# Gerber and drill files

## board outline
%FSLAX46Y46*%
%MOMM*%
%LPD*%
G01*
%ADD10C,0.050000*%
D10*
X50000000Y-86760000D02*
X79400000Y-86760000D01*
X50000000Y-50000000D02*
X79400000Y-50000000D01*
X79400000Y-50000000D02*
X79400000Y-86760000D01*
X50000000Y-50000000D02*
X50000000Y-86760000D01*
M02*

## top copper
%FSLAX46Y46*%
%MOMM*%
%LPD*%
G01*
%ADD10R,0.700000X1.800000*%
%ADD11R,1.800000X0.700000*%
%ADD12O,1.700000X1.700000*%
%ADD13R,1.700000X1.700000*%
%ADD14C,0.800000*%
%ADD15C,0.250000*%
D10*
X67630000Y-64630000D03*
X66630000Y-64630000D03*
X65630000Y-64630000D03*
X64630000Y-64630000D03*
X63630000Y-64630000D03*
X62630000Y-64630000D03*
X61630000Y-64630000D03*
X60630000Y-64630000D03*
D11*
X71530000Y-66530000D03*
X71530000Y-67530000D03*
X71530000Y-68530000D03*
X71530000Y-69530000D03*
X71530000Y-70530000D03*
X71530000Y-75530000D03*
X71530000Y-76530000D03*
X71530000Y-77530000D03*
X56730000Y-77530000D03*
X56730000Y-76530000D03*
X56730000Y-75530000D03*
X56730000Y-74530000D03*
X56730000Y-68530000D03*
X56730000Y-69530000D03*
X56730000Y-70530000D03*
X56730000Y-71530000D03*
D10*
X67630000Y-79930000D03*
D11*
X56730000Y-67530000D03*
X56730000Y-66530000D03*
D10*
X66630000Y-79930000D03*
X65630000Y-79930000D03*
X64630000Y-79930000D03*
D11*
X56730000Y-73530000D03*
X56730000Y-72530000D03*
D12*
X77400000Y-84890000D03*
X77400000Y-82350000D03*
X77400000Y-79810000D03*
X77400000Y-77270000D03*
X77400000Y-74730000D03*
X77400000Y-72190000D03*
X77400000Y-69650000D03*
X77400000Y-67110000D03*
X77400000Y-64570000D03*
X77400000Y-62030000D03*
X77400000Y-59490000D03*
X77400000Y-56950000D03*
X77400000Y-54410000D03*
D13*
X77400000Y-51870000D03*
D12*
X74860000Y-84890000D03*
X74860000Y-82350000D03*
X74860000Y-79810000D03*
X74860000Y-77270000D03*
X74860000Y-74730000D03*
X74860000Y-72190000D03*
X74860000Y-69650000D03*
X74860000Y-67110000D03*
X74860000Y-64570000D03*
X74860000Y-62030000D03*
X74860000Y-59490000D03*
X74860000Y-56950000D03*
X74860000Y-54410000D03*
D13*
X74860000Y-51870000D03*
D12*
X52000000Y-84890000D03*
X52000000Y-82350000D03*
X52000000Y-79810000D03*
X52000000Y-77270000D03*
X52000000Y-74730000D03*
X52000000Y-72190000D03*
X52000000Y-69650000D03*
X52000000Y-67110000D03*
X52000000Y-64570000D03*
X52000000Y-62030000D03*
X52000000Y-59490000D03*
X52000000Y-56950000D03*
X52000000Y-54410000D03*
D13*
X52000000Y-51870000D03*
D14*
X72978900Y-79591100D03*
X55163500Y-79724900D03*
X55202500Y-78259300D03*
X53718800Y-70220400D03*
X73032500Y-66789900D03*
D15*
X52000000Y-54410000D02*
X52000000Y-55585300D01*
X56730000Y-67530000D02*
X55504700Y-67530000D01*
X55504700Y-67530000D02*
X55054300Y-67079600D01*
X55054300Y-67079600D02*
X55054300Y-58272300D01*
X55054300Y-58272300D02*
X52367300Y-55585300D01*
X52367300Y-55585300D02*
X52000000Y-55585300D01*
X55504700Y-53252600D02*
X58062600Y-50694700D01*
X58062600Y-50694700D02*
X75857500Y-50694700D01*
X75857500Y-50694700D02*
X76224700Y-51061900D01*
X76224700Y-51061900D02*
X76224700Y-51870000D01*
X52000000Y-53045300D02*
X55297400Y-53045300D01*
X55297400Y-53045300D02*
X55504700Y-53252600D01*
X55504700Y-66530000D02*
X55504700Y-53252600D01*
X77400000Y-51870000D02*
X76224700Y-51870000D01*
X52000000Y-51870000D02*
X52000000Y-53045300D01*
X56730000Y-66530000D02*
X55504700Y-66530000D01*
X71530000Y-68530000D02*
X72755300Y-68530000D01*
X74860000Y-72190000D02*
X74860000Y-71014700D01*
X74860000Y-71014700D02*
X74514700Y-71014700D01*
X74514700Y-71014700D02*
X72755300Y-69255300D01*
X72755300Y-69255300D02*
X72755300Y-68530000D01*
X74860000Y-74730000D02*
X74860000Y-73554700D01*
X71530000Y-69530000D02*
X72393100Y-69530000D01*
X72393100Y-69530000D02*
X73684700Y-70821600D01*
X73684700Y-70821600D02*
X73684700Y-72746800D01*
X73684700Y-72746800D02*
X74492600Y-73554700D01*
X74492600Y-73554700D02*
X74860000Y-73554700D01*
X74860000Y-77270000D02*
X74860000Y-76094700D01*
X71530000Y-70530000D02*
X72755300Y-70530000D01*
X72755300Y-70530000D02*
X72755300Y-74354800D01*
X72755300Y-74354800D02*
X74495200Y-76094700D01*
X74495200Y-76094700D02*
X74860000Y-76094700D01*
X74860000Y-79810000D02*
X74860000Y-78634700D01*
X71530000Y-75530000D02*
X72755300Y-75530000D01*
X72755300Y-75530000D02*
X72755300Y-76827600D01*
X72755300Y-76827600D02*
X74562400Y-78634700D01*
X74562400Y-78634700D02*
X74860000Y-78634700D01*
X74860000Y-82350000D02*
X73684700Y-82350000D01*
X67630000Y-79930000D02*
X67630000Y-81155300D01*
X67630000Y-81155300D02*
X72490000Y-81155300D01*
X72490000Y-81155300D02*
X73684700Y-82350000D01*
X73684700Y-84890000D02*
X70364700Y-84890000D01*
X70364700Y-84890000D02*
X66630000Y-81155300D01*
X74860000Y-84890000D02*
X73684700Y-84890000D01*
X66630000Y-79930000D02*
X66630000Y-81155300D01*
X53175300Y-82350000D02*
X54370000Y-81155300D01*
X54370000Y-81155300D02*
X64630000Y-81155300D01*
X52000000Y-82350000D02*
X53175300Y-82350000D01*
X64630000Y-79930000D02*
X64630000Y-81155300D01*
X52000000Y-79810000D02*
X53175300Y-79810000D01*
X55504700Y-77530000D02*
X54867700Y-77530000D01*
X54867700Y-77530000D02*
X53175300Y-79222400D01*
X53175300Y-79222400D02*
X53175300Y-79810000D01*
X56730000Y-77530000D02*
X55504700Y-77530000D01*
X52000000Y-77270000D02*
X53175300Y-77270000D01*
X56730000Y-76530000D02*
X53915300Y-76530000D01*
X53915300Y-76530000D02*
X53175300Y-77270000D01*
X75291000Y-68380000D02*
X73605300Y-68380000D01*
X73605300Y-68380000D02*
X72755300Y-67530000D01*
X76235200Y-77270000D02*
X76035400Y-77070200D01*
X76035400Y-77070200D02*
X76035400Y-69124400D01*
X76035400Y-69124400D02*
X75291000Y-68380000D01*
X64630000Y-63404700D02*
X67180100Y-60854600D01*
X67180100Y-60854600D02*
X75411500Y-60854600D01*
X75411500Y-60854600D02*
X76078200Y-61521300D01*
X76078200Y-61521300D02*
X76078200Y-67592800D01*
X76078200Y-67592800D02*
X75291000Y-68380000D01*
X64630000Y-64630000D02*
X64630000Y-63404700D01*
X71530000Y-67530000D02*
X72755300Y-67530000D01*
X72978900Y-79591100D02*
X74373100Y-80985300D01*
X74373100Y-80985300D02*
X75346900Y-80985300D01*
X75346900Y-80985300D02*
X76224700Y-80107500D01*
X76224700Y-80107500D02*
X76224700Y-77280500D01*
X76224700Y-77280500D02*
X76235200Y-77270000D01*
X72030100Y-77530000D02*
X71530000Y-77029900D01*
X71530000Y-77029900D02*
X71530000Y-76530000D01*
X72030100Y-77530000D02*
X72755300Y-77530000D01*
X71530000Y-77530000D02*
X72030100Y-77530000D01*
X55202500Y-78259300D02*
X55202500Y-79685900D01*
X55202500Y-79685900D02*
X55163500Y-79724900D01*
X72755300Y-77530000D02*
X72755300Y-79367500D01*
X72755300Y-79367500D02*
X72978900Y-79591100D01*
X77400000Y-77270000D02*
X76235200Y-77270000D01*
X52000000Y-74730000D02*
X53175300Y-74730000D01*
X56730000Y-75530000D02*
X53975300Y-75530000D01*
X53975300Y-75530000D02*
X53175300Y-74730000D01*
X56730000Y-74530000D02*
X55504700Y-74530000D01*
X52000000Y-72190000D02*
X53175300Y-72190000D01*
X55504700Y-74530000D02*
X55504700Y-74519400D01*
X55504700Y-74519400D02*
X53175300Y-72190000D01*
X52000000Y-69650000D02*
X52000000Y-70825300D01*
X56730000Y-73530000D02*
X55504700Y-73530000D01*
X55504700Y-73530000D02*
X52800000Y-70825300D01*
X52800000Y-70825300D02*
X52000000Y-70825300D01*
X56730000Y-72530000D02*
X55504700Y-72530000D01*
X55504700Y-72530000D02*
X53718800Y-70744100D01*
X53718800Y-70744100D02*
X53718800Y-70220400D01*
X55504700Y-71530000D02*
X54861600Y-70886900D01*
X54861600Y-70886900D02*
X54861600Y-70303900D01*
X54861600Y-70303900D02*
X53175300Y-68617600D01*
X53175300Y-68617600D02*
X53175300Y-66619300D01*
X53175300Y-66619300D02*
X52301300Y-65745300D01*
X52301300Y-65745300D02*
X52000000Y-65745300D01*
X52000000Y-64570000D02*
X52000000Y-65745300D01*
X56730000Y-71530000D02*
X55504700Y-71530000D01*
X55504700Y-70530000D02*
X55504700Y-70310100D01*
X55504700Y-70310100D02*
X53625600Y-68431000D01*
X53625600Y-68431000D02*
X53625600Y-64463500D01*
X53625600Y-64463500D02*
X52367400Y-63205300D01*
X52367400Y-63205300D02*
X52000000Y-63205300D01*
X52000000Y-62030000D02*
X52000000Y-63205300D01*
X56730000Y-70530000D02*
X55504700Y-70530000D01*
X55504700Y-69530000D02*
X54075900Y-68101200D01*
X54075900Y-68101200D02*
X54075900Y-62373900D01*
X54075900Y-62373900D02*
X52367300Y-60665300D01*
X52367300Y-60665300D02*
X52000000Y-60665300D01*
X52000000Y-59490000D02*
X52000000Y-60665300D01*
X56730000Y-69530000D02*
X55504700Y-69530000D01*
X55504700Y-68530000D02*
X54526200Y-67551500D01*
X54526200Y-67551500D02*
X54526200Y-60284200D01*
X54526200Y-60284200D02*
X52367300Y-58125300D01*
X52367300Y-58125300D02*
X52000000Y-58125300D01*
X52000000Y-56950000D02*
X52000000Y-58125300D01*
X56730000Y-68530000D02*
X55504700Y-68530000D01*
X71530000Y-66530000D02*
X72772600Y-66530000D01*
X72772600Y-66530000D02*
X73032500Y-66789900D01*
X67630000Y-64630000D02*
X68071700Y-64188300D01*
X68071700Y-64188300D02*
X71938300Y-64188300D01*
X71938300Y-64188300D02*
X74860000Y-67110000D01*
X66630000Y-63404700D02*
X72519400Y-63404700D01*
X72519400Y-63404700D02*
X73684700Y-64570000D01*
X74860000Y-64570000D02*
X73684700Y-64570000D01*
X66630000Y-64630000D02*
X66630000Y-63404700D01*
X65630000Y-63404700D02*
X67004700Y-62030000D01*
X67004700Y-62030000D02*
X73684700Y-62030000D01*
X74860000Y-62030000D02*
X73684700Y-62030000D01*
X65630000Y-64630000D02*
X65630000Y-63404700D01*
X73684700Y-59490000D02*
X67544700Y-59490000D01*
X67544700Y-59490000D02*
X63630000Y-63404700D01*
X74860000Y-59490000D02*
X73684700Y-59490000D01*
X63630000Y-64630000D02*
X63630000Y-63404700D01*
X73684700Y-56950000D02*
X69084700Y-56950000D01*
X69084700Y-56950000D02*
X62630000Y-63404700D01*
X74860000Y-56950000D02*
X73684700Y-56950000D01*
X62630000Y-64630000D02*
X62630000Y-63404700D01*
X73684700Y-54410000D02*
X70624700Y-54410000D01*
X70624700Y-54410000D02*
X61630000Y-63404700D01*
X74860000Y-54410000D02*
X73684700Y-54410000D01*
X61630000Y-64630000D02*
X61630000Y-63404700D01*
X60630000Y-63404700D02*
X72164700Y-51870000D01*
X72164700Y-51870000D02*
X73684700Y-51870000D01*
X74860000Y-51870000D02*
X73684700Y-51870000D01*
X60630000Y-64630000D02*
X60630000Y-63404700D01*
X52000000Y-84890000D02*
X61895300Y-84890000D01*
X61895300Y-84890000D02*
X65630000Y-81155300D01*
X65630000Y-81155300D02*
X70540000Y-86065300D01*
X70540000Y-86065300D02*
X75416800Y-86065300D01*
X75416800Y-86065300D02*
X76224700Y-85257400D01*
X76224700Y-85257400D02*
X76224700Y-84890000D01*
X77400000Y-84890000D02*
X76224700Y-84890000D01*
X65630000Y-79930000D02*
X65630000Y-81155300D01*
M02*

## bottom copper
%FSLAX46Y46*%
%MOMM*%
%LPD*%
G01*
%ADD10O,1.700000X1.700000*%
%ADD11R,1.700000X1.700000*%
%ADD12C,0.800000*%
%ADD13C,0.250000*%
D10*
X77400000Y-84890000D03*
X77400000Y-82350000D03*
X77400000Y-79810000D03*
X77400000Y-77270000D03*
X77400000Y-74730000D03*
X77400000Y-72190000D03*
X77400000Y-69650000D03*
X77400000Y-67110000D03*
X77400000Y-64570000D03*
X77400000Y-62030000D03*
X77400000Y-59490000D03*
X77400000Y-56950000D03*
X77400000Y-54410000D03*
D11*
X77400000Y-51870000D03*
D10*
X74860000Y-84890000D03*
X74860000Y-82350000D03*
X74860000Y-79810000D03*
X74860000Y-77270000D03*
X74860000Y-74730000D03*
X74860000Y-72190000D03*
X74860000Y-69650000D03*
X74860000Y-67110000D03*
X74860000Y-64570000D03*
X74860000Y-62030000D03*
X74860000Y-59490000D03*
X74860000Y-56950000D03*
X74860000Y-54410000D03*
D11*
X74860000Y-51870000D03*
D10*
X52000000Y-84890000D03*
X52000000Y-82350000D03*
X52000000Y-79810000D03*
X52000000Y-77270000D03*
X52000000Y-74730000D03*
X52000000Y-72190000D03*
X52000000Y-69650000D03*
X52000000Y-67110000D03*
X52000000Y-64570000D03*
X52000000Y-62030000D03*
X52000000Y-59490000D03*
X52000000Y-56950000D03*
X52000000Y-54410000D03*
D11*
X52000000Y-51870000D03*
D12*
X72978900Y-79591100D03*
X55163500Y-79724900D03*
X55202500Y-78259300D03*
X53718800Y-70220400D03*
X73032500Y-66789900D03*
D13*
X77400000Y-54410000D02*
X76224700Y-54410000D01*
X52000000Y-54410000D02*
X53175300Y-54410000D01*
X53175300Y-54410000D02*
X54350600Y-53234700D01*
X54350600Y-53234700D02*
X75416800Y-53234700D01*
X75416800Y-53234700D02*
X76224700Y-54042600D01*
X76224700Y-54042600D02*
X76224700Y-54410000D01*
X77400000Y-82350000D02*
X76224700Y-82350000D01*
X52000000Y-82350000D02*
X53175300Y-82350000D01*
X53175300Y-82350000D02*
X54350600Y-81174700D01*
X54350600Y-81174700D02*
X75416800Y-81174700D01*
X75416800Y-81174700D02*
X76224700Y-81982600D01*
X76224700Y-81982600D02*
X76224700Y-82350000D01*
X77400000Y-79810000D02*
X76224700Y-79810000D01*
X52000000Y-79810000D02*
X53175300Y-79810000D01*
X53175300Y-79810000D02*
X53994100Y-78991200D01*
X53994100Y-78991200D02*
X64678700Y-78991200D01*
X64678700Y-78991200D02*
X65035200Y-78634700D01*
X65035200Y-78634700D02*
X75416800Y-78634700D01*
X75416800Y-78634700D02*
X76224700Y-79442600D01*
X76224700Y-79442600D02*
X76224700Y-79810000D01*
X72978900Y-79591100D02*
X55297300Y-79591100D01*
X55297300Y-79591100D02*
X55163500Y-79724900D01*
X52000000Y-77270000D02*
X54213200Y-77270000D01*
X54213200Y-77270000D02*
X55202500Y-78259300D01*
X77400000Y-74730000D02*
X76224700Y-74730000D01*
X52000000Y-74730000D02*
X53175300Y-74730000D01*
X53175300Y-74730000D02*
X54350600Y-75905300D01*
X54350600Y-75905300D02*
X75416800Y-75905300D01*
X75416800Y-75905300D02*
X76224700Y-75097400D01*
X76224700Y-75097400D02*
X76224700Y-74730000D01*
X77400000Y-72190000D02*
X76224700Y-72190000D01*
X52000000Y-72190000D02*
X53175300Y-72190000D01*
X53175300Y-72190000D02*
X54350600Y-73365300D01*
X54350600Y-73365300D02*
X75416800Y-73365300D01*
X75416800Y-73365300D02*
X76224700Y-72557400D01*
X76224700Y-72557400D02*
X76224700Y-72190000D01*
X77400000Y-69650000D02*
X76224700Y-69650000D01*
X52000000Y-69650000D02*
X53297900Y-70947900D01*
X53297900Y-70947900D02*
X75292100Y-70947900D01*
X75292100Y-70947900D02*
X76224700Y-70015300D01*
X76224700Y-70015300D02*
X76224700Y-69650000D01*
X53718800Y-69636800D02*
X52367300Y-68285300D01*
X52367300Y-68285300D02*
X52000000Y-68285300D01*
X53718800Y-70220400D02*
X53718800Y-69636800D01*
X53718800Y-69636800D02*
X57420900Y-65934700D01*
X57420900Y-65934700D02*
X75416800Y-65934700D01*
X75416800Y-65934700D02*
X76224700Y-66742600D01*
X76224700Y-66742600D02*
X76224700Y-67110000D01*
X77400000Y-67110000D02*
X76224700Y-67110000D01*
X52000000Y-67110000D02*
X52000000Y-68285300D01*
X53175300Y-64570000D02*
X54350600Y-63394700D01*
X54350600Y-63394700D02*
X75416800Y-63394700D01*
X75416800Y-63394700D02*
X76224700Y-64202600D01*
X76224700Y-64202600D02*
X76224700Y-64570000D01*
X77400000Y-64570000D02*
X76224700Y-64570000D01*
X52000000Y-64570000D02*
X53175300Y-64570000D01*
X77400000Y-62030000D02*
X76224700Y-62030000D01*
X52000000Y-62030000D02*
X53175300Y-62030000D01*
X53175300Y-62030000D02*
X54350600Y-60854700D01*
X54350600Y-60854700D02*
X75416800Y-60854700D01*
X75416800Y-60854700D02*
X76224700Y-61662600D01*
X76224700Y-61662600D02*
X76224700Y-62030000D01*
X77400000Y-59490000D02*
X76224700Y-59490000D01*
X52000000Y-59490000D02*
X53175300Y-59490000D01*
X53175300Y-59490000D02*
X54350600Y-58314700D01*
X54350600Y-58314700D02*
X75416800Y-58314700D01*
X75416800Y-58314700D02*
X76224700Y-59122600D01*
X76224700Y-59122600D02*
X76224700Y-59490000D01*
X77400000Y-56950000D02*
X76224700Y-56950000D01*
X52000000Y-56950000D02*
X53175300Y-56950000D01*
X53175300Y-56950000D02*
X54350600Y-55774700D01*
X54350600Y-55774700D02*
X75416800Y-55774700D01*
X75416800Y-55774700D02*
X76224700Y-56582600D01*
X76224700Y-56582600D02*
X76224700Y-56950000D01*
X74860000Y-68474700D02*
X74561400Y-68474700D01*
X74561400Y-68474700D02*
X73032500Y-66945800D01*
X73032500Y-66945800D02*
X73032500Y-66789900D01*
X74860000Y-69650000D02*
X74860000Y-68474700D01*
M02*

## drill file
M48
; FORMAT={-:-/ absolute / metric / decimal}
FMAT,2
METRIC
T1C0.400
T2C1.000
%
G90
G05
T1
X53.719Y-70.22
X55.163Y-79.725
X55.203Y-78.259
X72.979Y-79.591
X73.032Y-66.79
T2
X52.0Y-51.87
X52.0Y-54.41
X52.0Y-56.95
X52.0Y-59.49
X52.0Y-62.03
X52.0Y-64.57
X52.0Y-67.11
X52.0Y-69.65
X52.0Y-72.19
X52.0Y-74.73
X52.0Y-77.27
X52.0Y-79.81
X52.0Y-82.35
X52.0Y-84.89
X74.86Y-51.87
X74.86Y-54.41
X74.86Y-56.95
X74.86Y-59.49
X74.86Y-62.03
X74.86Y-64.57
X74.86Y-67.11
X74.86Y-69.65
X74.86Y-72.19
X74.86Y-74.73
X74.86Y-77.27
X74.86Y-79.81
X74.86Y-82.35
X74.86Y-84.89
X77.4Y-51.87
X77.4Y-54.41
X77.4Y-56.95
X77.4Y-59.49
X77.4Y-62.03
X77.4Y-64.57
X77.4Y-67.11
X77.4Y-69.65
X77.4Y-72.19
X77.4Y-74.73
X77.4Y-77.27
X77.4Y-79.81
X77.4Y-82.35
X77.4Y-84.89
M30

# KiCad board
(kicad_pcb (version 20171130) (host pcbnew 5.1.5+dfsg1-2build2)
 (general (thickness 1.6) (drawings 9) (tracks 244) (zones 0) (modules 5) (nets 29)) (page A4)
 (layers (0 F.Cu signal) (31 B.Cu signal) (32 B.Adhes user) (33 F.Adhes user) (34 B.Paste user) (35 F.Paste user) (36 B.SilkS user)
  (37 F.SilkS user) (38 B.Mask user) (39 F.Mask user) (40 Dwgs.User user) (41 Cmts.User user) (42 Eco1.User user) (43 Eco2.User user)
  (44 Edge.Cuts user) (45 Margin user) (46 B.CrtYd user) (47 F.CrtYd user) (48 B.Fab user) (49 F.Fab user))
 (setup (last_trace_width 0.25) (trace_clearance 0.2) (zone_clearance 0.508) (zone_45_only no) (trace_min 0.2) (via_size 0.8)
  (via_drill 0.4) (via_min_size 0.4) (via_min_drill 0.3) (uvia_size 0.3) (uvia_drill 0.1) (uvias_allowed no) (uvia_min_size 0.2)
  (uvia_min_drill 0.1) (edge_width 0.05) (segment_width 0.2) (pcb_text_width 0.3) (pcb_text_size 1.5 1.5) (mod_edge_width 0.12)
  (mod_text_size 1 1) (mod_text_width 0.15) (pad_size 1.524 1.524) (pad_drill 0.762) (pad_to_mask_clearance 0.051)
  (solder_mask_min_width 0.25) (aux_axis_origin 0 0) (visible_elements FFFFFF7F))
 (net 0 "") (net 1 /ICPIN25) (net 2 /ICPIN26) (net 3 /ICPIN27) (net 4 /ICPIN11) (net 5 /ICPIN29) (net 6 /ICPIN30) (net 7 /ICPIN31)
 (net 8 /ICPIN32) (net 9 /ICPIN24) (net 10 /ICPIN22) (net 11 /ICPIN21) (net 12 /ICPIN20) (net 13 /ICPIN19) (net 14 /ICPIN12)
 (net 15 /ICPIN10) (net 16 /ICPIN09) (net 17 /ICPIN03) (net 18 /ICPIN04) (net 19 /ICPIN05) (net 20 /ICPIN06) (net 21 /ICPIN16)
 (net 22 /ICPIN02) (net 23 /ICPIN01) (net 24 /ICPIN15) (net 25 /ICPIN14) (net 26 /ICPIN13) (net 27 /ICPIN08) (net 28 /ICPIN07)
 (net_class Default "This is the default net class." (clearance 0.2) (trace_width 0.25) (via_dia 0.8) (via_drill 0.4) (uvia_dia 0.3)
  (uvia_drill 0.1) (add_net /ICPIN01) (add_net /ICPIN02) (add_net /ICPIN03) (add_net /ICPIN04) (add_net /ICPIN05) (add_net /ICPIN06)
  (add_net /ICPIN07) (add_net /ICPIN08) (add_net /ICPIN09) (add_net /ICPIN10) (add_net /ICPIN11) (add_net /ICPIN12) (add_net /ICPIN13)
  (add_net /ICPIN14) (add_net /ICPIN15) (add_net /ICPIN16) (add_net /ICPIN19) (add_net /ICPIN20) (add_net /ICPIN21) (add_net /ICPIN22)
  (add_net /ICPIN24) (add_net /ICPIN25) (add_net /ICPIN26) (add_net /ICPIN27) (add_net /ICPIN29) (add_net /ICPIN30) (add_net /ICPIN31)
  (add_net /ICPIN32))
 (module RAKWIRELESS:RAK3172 (layer F.Cu) (at 64.13 72.28)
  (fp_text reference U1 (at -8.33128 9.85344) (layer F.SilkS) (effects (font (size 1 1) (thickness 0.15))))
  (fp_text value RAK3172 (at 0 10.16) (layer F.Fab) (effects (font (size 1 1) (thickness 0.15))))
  (pad 25 smd rect (at 3.5 -7.65 270) (size 1.8 0.7) (layers F.Cu F.Paste F.Mask) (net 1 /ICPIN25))
  (pad 26 smd rect (at 2.5 -7.65 270) (size 1.8 0.7) (layers F.Cu F.Paste F.Mask) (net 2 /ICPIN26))
  (pad 27 smd rect (at 1.5 -7.65 270) (size 1.8 0.7) (layers F.Cu F.Paste F.Mask) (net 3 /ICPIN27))
  (pad 28 smd rect (at 0.5 -7.65 270) (size 1.8 0.7) (layers F.Cu F.Paste F.Mask) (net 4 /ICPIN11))
  (pad 29 smd rect (at -0.5 -7.65 270) (size 1.8 0.7) (layers F.Cu F.Paste F.Mask) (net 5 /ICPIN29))
  (pad 30 smd rect (at -1.5 -7.65 270) (size 1.8 0.7) (layers F.Cu F.Paste F.Mask) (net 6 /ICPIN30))
  (pad 31 smd rect (at -2.5 -7.65 270) (size 1.8 0.7) (layers F.Cu F.Paste F.Mask) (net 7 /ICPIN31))
  (pad 32 smd rect (at -3.5 -7.65 270) (size 1.8 0.7) (layers F.Cu F.Paste F.Mask) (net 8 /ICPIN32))
  (pad 24 smd rect (at 7.4 -5.75) (size 1.8 0.7) (layers F.Cu F.Paste F.Mask) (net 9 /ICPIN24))
  (pad 23 smd rect (at 7.4 -4.75) (size 1.8 0.7) (layers F.Cu F.Paste F.Mask) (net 4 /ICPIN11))
  (pad 22 smd rect (at 7.4 -3.75) (size 1.8 0.7) (layers F.Cu F.Paste F.Mask) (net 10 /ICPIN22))
  (pad 21 smd rect (at 7.4 -2.75) (size 1.8 0.7) (layers F.Cu F.Paste F.Mask) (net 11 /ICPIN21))
  (pad 20 smd rect (at 7.4 -1.75) (size 1.8 0.7) (layers F.Cu F.Paste F.Mask) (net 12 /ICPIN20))
  (pad 19 smd rect (at 7.4 3.25) (size 1.8 0.7) (layers F.Cu F.Paste F.Mask) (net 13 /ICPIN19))
  (pad 18 smd rect (at 7.4 4.25) (size 1.8 0.7) (layers F.Cu F.Paste F.Mask) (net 4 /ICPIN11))
  (pad 17 smd rect (at 7.4 5.25) (size 1.8 0.7) (layers F.Cu F.Paste F.Mask) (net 4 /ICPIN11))
  (pad 12 smd rect (at -7.4 5.25) (size 1.8 0.7) (layers F.Cu F.Paste F.Mask) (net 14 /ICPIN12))
  (pad 11 smd rect (at -7.4 4.25) (size 1.8 0.7) (layers F.Cu F.Paste F.Mask) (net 4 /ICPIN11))
  (pad 10 smd rect (at -7.4 3.25) (size 1.8 0.7) (layers F.Cu F.Paste F.Mask) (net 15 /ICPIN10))
  (pad 9 smd rect (at -7.4 2.25) (size 1.8 0.7) (layers F.Cu F.Paste F.Mask) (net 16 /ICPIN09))
  (pad 3 smd rect (at -7.4 -3.75) (size 1.8 0.7) (layers F.Cu F.Paste F.Mask) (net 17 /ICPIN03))
  (pad 4 smd rect (at -7.4 -2.75) (size 1.8 0.7) (layers F.Cu F.Paste F.Mask) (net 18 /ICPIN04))
  (pad 5 smd rect (at -7.4 -1.75) (size 1.8 0.7) (layers F.Cu F.Paste F.Mask) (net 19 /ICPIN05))
  (pad 6 smd rect (at -7.4 -0.75) (size 1.8 0.7) (layers F.Cu F.Paste F.Mask) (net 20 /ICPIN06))
  (pad 16 smd rect (at 3.5 7.65 90) (size 1.8 0.7) (layers F.Cu F.Paste F.Mask) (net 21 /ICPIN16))
  (pad 2 smd rect (at -7.4 -4.75) (size 1.8 0.7) (layers F.Cu F.Paste F.Mask) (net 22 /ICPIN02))
  (pad 1 smd rect (at -7.4 -5.75) (size 1.8 0.7) (layers F.Cu F.Paste F.Mask) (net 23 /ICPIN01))
  (pad 15 smd rect (at 2.5 7.65 90) (size 1.8 0.7) (layers F.Cu F.Paste F.Mask) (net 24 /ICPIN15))
  (pad 14 smd rect (at 1.5 7.65 90) (size 1.8 0.7) (layers F.Cu F.Paste F.Mask) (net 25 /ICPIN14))
  (pad 13 smd rect (at 0.5 7.65 270) (size 1.8 0.7) (layers F.Cu F.Paste F.Mask) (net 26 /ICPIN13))
  (pad 8 smd rect (at -7.4 1.25) (size 1.8 0.7) (layers F.Cu F.Paste F.Mask) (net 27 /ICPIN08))
  (pad 7 smd rect (at -7.4 0.25) (size 1.8 0.7) (layers F.Cu F.Paste F.Mask) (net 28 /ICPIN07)))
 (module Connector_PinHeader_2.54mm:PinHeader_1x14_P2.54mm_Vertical (layer F.Cu) (at 77.4 51.87)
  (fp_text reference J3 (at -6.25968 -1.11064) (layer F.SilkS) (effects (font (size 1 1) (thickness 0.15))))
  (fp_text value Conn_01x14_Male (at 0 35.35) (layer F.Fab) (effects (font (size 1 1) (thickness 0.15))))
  (pad 14 thru_hole oval (at 0 33.02) (size 1.7 1.7) (drill 1) (layers *.Cu *.Mask) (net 25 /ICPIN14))
  (pad 13 thru_hole oval (at 0 30.48) (size 1.7 1.7) (drill 1) (layers *.Cu *.Mask) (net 26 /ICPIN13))
  (pad 12 thru_hole oval (at 0 27.94) (size 1.7 1.7) (drill 1) (layers *.Cu *.Mask) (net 14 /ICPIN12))
  (pad 11 thru_hole oval (at 0 25.4) (size 1.7 1.7) (drill 1) (layers *.Cu *.Mask) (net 4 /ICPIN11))
  (pad 10 thru_hole oval (at 0 22.86) (size 1.7 1.7) (drill 1) (layers *.Cu *.Mask) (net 15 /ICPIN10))
  (pad 9 thru_hole oval (at 0 20.32) (size 1.7 1.7) (drill 1) (layers *.Cu *.Mask) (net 16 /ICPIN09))
  (pad 8 thru_hole oval (at 0 17.78) (size 1.7 1.7) (drill 1) (layers *.Cu *.Mask) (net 27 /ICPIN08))
  (pad 7 thru_hole oval (at 0 15.24) (size 1.7 1.7) (drill 1) (layers *.Cu *.Mask) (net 28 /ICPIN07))
  (pad 6 thru_hole oval (at 0 12.7) (size 1.7 1.7) (drill 1) (layers *.Cu *.Mask) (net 20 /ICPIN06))
  (pad 5 thru_hole oval (at 0 10.16) (size 1.7 1.7) (drill 1) (layers *.Cu *.Mask) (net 19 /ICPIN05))
  (pad 4 thru_hole oval (at 0 7.62) (size 1.7 1.7) (drill 1) (layers *.Cu *.Mask) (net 18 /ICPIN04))
  (pad 3 thru_hole oval (at 0 5.08) (size 1.7 1.7) (drill 1) (layers *.Cu *.Mask) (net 17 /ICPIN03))
  (pad 2 thru_hole oval (at 0 2.54) (size 1.7 1.7) (drill 1) (layers *.Cu *.Mask) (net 22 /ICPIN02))
  (pad 1 thru_hole rect (at 0 0) (size 1.7 1.7) (drill 1) (layers *.Cu *.Mask) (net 23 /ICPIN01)))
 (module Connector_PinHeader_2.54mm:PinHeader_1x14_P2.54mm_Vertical (layer F.Cu) (at 74.86 51.87)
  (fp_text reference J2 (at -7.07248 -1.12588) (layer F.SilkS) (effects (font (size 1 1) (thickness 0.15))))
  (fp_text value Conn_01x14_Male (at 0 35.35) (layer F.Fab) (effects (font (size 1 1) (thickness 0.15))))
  (pad 14 thru_hole oval (at 0 33.02) (size 1.7 1.7) (drill 1) (layers *.Cu *.Mask) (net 24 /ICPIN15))
  (pad 13 thru_hole oval (at 0 30.48) (size 1.7 1.7) (drill 1) (layers *.Cu *.Mask) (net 21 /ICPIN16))
  (pad 12 thru_hole oval (at 0 27.94) (size 1.7 1.7) (drill 1) (layers *.Cu *.Mask) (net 13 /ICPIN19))
  (pad 11 thru_hole oval (at 0 25.4) (size 1.7 1.7) (drill 1) (layers *.Cu *.Mask) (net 12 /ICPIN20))
  (pad 10 thru_hole oval (at 0 22.86) (size 1.7 1.7) (drill 1) (layers *.Cu *.Mask) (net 11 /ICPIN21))
  (pad 9 thru_hole oval (at 0 20.32) (size 1.7 1.7) (drill 1) (layers *.Cu *.Mask) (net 10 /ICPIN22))
  (pad 8 thru_hole oval (at 0 17.78) (size 1.7 1.7) (drill 1) (layers *.Cu *.Mask) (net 9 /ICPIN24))
  (pad 7 thru_hole oval (at 0 15.24) (size 1.7 1.7) (drill 1) (layers *.Cu *.Mask) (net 1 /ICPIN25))
  (pad 6 thru_hole oval (at 0 12.7) (size 1.7 1.7) (drill 1) (layers *.Cu *.Mask) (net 2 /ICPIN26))
  (pad 5 thru_hole oval (at 0 10.16) (size 1.7 1.7) (drill 1) (layers *.Cu *.Mask) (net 3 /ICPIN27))
  (pad 4 thru_hole oval (at 0 7.62) (size 1.7 1.7) (drill 1) (layers *.Cu *.Mask) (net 5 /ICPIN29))
  (pad 3 thru_hole oval (at 0 5.08) (size 1.7 1.7) (drill 1) (layers *.Cu *.Mask) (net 6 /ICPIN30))
  (pad 2 thru_hole oval (at 0 2.54) (size 1.7 1.7) (drill 1) (layers *.Cu *.Mask) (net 7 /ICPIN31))
  (pad 1 thru_hole rect (at 0 0) (size 1.7 1.7) (drill 1) (layers *.Cu *.Mask) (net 8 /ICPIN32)))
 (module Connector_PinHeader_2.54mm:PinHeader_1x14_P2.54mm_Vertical (layer F.Cu) (at 52 51.87)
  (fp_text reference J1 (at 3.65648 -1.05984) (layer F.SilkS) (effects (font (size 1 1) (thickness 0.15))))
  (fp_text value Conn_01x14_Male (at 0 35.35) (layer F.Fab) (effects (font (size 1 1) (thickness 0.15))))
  (pad 14 thru_hole oval (at 0 33.02) (size 1.7 1.7) (drill 1) (layers *.Cu *.Mask) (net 25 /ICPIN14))
  (pad 13 thru_hole oval (at 0 30.48) (size 1.7 1.7) (drill 1) (layers *.Cu *.Mask) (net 26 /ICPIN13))
  (pad 12 thru_hole oval (at 0 27.94) (size 1.7 1.7) (drill 1) (layers *.Cu *.Mask) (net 14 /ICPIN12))
  (pad 11 thru_hole oval (at 0 25.4) (size 1.7 1.7) (drill 1) (layers *.Cu *.Mask) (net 4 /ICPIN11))
  (pad 10 thru_hole oval (at 0 22.86) (size 1.7 1.7) (drill 1) (layers *.Cu *.Mask) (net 15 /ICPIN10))
  (pad 9 thru_hole oval (at 0 20.32) (size 1.7 1.7) (drill 1) (layers *.Cu *.Mask) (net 16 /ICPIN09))
  (pad 8 thru_hole oval (at 0 17.78) (size 1.7 1.7) (drill 1) (layers *.Cu *.Mask) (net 27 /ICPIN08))
  (pad 7 thru_hole oval (at 0 15.24) (size 1.7 1.7) (drill 1) (layers *.Cu *.Mask) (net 28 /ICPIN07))
  (pad 6 thru_hole oval (at 0 12.7) (size 1.7 1.7) (drill 1) (layers *.Cu *.Mask) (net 20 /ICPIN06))
  (pad 5 thru_hole oval (at 0 10.16) (size 1.7 1.7) (drill 1) (layers *.Cu *.Mask) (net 19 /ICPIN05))
  (pad 4 thru_hole oval (at 0 7.62) (size 1.7 1.7) (drill 1) (layers *.Cu *.Mask) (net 18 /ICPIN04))
  (pad 3 thru_hole oval (at 0 5.08) (size 1.7 1.7) (drill 1) (layers *.Cu *.Mask) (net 17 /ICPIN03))
  (pad 2 thru_hole oval (at 0 2.54) (size 1.7 1.7) (drill 1) (layers *.Cu *.Mask) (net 22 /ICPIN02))
  (pad 1 thru_hole rect (at 0 0) (size 1.7 1.7) (drill 1) (layers *.Cu *.Mask) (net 23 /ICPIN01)))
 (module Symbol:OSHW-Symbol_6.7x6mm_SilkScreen (layer F.Cu) (at 60.7822 56.03748)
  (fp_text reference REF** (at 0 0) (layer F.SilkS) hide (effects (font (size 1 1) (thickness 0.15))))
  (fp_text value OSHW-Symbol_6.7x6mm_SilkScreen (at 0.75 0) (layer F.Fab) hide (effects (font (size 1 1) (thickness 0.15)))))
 (gr_line (start 50 86.76) (end 79.4 86.76) (layer Edge.Cuts) (width 0.05))
 (gr_line (start 50 50) (end 79.4 50) (layer Edge.Cuts) (width 0.05))
 (gr_line (start 79.4 50) (end 79.4 86.76) (layer Edge.Cuts) (width 0.05))
 (gr_line (start 50 50) (end 50 86.76) (layer Edge.Cuts) (width 0.05))
 (segment (start 52 54.41) (end 52 55.5853) (width 0.25) (layer F.Cu) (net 22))
 (segment (start 56.73 67.53) (end 55.5047 67.53) (width 0.25) (layer F.Cu) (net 22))
 (segment (start 55.5047 67.53) (end 55.0543 67.0796) (width 0.25) (layer F.Cu) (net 22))
 (segment (start 55.0543 67.0796) (end 55.0543 58.2723) (width 0.25) (layer F.Cu) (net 22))
 (segment (start 55.0543 58.2723) (end 52.3673 55.5853) (width 0.25) (layer F.Cu) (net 22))
 (segment (start 52.3673 55.5853) (end 52 55.5853) (width 0.25) (layer F.Cu) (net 22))
 (segment (start 77.4 54.41) (end 76.2247 54.41) (width 0.25) (layer B.Cu) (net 22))
 (segment (start 52 54.41) (end 53.1753 54.41) (width 0.25) (layer B.Cu) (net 22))
 (segment (start 53.1753 54.41) (end 54.3506 53.2347) (width 0.25) (layer B.Cu) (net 22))
 (segment (start 54.3506 53.2347) (end 75.4168 53.2347) (width 0.25) (layer B.Cu) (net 22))
 (segment (start 75.4168 53.2347) (end 76.2247 54.0426) (width 0.25) (layer B.Cu) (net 22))
 (segment (start 76.2247 54.0426) (end 76.2247 54.41) (width 0.25) (layer B.Cu) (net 22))
 (segment (start 55.5047 53.2526) (end 58.0626 50.6947) (width 0.25) (layer F.Cu) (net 23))
 (segment (start 58.0626 50.6947) (end 75.8575 50.6947) (width 0.25) (layer F.Cu) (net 23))
 (segment (start 75.8575 50.6947) (end 76.2247 51.0619) (width 0.25) (layer F.Cu) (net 23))
 (segment (start 76.2247 51.0619) (end 76.2247 51.87) (width 0.25) (layer F.Cu) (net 23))
 (segment (start 52 53.0453) (end 55.2974 53.0453) (width 0.25) (layer F.Cu) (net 23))
 (segment (start 55.2974 53.0453) (end 55.5047 53.2526) (width 0.25) (layer F.Cu) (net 23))
 (segment (start 55.5047 66.53) (end 55.5047 53.2526) (width 0.25) (layer F.Cu) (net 23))
 (segment (start 77.4 51.87) (end 76.2247 51.87) (width 0.25) (layer F.Cu) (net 23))
 (segment (start 52 51.87) (end 52 53.0453) (width 0.25) (layer F.Cu) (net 23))
 (segment (start 56.73 66.53) (end 55.5047 66.53) (width 0.25) (layer F.Cu) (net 23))
 (segment (start 71.53 68.53) (end 72.7553 68.53) (width 0.25) (layer F.Cu) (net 10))
 (segment (start 74.86 72.19) (end 74.86 71.0147) (width 0.25) (layer F.Cu) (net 10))
 (segment (start 74.86 71.0147) (end 74.5147 71.0147) (width 0.25) (layer F.Cu) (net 10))
 (segment (start 74.5147 71.0147) (end 72.7553 69.2553) (width 0.25) (layer F.Cu) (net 10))
 (segment (start 72.7553 69.2553) (end 72.7553 68.53) (width 0.25) (layer F.Cu) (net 10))
 (segment (start 74.86 74.73) (end 74.86 73.5547) (width 0.25) (layer F.Cu) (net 11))
 (segment (start 71.53 69.53) (end 72.3931 69.53) (width 0.25) (layer F.Cu) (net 11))
 (segment (start 72.3931 69.53) (end 73.6847 70.8216) (width 0.25) (layer F.Cu) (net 11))
 (segment (start 73.6847 70.8216) (end 73.6847 72.7468) (width 0.25) (layer F.Cu) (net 11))
 (segment (start 73.6847 72.7468) (end 74.4926 73.5547) (width 0.25) (layer F.Cu) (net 11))
 (segment (start 74.4926 73.5547) (end 74.86 73.5547) (width 0.25) (layer F.Cu) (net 11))
 (segment (start 74.86 77.27) (end 74.86 76.0947) (width 0.25) (layer F.Cu) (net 12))
 (segment (start 71.53 70.53) (end 72.7553 70.53) (width 0.25) (layer F.Cu) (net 12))
 (segment (start 72.7553 70.53) (end 72.7553 74.3548) (width 0.25) (layer F.Cu) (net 12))
 (segment (start 72.7553 74.3548) (end 74.4952 76.0947) (width 0.25) (layer F.Cu) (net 12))
 (segment (start 74.4952 76.0947) (end 74.86 76.0947) (width 0.25) (layer F.Cu) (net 12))
 (segment (start 74.86 79.81) (end 74.86 78.6347) (width 0.25) (layer F.Cu) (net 13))
 (segment (start 71.53 75.53) (end 72.7553 75.53) (width 0.25) (layer F.Cu) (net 13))
 (segment (start 72.7553 75.53) (end 72.7553 76.8276) (width 0.25) (layer F.Cu) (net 13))
 (segment (start 72.7553 76.8276) (end 74.5624 78.6347) (width 0.25) (layer F.Cu) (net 13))
 (segment (start 74.5624 78.6347) (end 74.86 78.6347) (width 0.25) (layer F.Cu) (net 13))
 (segment (start 74.86 82.35) (end 73.6847 82.35) (width 0.25) (layer F.Cu) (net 21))
 (segment (start 67.63 79.93) (end 67.63 81.1553) (width 0.25) (layer F.Cu) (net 21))
 (segment (start 67.63 81.1553) (end 72.49 81.1553) (width 0.25) (layer F.Cu) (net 21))
 (segment (start 72.49 81.1553) (end 73.6847 82.35) (width 0.25) (layer F.Cu) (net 21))
 (segment (start 73.6847 84.89) (end 70.3647 84.89) (width 0.25) (layer F.Cu) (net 24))
 (segment (start 70.3647 84.89) (end 66.63 81.1553) (width 0.25) (layer F.Cu) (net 24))
 (segment (start 74.86 84.89) (end 73.6847 84.89) (width 0.25) (layer F.Cu) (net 24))
 (segment (start 66.63 79.93) (end 66.63 81.1553) (width 0.25) (layer F.Cu) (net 24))
 (segment (start 77.4 82.35) (end 76.2247 82.35) (width 0.25) (layer B.Cu) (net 26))
 (segment (start 52 82.35) (end 53.1753 82.35) (width 0.25) (layer B.Cu) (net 26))
 (segment (start 53.1753 82.35) (end 54.3506 81.1747) (width 0.25) (layer B.Cu) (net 26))
 (segment (start 54.3506 81.1747) (end 75.4168 81.1747) (width 0.25) (layer B.Cu) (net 26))
 (segment (start 75.4168 81.1747) (end 76.2247 81.9826) (width 0.25) (layer B.Cu) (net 26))
 (segment (start 76.2247 81.9826) (end 76.2247 82.35) (width 0.25) (layer B.Cu) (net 26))
 (segment (start 53.1753 82.35) (end 54.37 81.1553) (width 0.25) (layer F.Cu) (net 26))
 (segment (start 54.37 81.1553) (end 64.63 81.1553) (width 0.25) (layer F.Cu) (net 26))
 (segment (start 52 82.35) (end 53.1753 82.35) (width 0.25) (layer F.Cu) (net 26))
 (segment (start 64.63 79.93) (end 64.63 81.1553) (width 0.25) (layer F.Cu) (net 26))
 (segment (start 77.4 79.81) (end 76.2247 79.81) (width 0.25) (layer B.Cu) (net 14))
 (segment (start 52 79.81) (end 53.1753 79.81) (width 0.25) (layer B.Cu) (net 14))
 (segment (start 53.1753 79.81) (end 53.9941 78.9912) (width 0.25) (layer B.Cu) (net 14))
 (segment (start 53.9941 78.9912) (end 64.6787 78.9912) (width 0.25) (layer B.Cu) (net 14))
 (segment (start 64.6787 78.9912) (end 65.0352 78.6347) (width 0.25) (layer B.Cu) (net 14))
 (segment (start 65.0352 78.6347) (end 75.4168 78.6347) (width 0.25) (layer B.Cu) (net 14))
 (segment (start 75.4168 78.6347) (end 76.2247 79.4426) (width 0.25) (layer B.Cu) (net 14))
 (segment (start 76.2247 79.4426) (end 76.2247 79.81) (width 0.25) (layer B.Cu) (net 14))
 (segment (start 52 79.81) (end 53.1753 79.81) (width 0.25) (layer F.Cu) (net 14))
 (segment (start 55.5047 77.53) (end 54.8677 77.53) (width 0.25) (layer F.Cu) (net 14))
 (segment (start 54.8677 77.53) (end 53.1753 79.2224) (width 0.25) (layer F.Cu) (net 14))
 (segment (start 53.1753 79.2224) (end 53.1753 79.81) (width 0.25) (layer F.Cu) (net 14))
 (segment (start 56.73 77.53) (end 55.5047 77.53) (width 0.25) (layer F.Cu) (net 14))
 (segment (start 52 77.27) (end 53.1753 77.27) (width 0.25) (layer F.Cu) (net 4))
 (segment (start 56.73 76.53) (end 53.9153 76.53) (width 0.25) (layer F.Cu) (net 4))
 (segment (start 53.9153 76.53) (end 53.1753 77.27) (width 0.25) (layer F.Cu) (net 4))
 (segment (start 75.291 68.38) (end 73.6053 68.38) (width 0.25) (layer F.Cu) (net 4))
 (segment (start 73.6053 68.38) (end 72.7553 67.53) (width 0.25) (layer F.Cu) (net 4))
 (segment (start 76.2352 77.27) (end 76.0354 77.0702) (width 0.25) (layer F.Cu) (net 4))
 (segment (start 76.0354 77.0702) (end 76.0354 69.1244) (width 0.25) (layer F.Cu) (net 4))
 (segment (start 76.0354 69.1244) (end 75.291 68.38) (width 0.25) (layer F.Cu) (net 4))
 (segment (start 64.63 63.4047) (end 67.1801 60.8546) (width 0.25) (layer F.Cu) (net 4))
 (segment (start 67.1801 60.8546) (end 75.4115 60.8546) (width 0.25) (layer F.Cu) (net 4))
 (segment (start 75.4115 60.8546) (end 76.0782 61.5213) (width 0.25) (layer F.Cu) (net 4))
 (segment (start 76.0782 61.5213) (end 76.0782 67.5928) (width 0.25) (layer F.Cu) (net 4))
 (segment (start 76.0782 67.5928) (end 75.291 68.38) (width 0.25) (layer F.Cu) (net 4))
 (segment (start 64.63 64.63) (end 64.63 63.4047) (width 0.25) (layer F.Cu) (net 4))
 (segment (start 71.53 67.53) (end 72.7553 67.53) (width 0.25) (layer F.Cu) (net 4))
 (segment (start 72.9789 79.5911) (end 74.3731 80.9853) (width 0.25) (layer F.Cu) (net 4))
 (segment (start 74.3731 80.9853) (end 75.3469 80.9853) (width 0.25) (layer F.Cu) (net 4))
 (segment (start 75.3469 80.9853) (end 76.2247 80.1075) (width 0.25) (layer F.Cu) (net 4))
 (segment (start 76.2247 80.1075) (end 76.2247 77.2805) (width 0.25) (layer F.Cu) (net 4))
 (segment (start 76.2247 77.2805) (end 76.2352 77.27) (width 0.25) (layer F.Cu) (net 4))
 (segment (start 72.0301 77.53) (end 71.53 77.0299) (width 0.25) (layer F.Cu) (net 4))
 (segment (start 71.53 77.0299) (end 71.53 76.53) (width 0.25) (layer F.Cu) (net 4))
 (segment (start 72.0301 77.53) (end 72.7553 77.53) (width 0.25) (layer F.Cu) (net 4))
 (segment (start 71.53 77.53) (end 72.0301 77.53) (width 0.25) (layer F.Cu) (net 4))
 (segment (start 55.2025 78.2593) (end 55.2025 79.6859) (width 0.25) (layer F.Cu) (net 4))
 (segment (start 55.2025 79.6859) (end 55.1635 79.7249) (width 0.25) (layer F.Cu) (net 4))
 (segment (start 72.9789 79.5911) (end 55.2973 79.5911) (width 0.25) (layer B.Cu) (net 4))
 (segment (start 55.2973 79.5911) (end 55.1635 79.7249) (width 0.25) (layer B.Cu) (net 4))
 (segment (start 72.7553 77.53) (end 72.7553 79.3675) (width 0.25) (layer F.Cu) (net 4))
 (segment (start 72.7553 79.3675) (end 72.9789 79.5911) (width 0.25) (layer F.Cu) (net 4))
 (segment (start 52 77.27) (end 54.2132 77.27) (width 0.25) (layer B.Cu) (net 4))
 (segment (start 54.2132 77.27) (end 55.2025 78.2593) (width 0.25) (layer B.Cu) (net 4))
 (segment (start 77.4 77.27) (end 76.2352 77.27) (width 0.25) (layer F.Cu) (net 4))
 (via (at 72.9789 79.5911) (size 0.8) (layers F.Cu B.Cu) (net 4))
 (via (at 55.1635 79.7249) (size 0.8) (layers F.Cu B.Cu) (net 4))
 (via (at 55.2025 78.2593) (size 0.8) (layers F.Cu B.Cu) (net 4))
 (segment (start 52 74.73) (end 53.1753 74.73) (width 0.25) (layer F.Cu) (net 15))
 (segment (start 56.73 75.53) (end 53.9753 75.53) (width 0.25) (layer F.Cu) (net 15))
 (segment (start 53.9753 75.53) (end 53.1753 74.73) (width 0.25) (layer F.Cu) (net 15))
 (segment (start 77.4 74.73) (end 76.2247 74.73) (width 0.25) (layer B.Cu) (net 15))
 (segment (start 52 74.73) (end 53.1753 74.73) (width 0.25) (layer B.Cu) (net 15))
 (segment (start 53.1753 74.73) (end 54.3506 75.9053) (width 0.25) (layer B.Cu) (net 15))
 (segment (start 54.3506 75.9053) (end 75.4168 75.9053) (width 0.25) (layer B.Cu) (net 15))
 (segment (start 75.4168 75.9053) (end 76.2247 75.0974) (width 0.25) (layer B.Cu) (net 15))
 (segment (start 76.2247 75.0974) (end 76.2247 74.73) (width 0.25) (layer B.Cu) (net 15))
 (segment (start 77.4 72.19) (end 76.2247 72.19) (width 0.25) (layer B.Cu) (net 16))
 (segment (start 52 72.19) (end 53.1753 72.19) (width 0.25) (layer B.Cu) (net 16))
 (segment (start 53.1753 72.19) (end 54.3506 73.3653) (width 0.25) (layer B.Cu) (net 16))
 (segment (start 54.3506 73.3653) (end 75.4168 73.3653) (width 0.25) (layer B.Cu) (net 16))
 (segment (start 75.4168 73.3653) (end 76.2247 72.5574) (width 0.25) (layer B.Cu) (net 16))
 (segment (start 76.2247 72.5574) (end 76.2247 72.19) (width 0.25) (layer B.Cu) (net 16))
 (segment (start 56.73 74.53) (end 55.5047 74.53) (width 0.25) (layer F.Cu) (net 16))
 (segment (start 52 72.19) (end 53.1753 72.19) (width 0.25) (layer F.Cu) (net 16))
 (segment (start 55.5047 74.53) (end 55.5047 74.5194) (width 0.25) (layer F.Cu) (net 16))
 (segment (start 55.5047 74.5194) (end 53.1753 72.19) (width 0.25) (layer F.Cu) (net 16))
 (segment (start 77.4 69.65) (end 76.2247 69.65) (width 0.25) (layer B.Cu) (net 27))
 (segment (start 52 69.65) (end 53.2979 70.9479) (width 0.25) (layer B.Cu) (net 27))
 (segment (start 53.2979 70.9479) (end 75.2921 70.9479) (width 0.25) (layer B.Cu) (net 27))
 (segment (start 75.2921 70.9479) (end 76.2247 70.0153) (width 0.25) (layer B.Cu) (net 27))
 (segment (start 76.2247 70.0153) (end 76.2247 69.65) (width 0.25) (layer B.Cu) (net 27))
 (segment (start 52 69.65) (end 52 70.8253) (width 0.25) (layer F.Cu) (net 27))
 (segment (start 56.73 73.53) (end 55.5047 73.53) (width 0.25) (layer F.Cu) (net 27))
 (segment (start 55.5047 73.53) (end 52.8 70.8253) (width 0.25) (layer F.Cu) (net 27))
 (segment (start 52.8 70.8253) (end 52 70.8253) (width 0.25) (layer F.Cu) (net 27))
 (segment (start 53.7188 69.6368) (end 52.3673 68.2853) (width 0.25) (layer B.Cu) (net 28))
 (segment (start 52.3673 68.2853) (end 52 68.2853) (width 0.25) (layer B.Cu) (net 28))
 (segment (start 53.7188 70.2204) (end 53.7188 69.6368) (width 0.25) (layer B.Cu) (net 28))
 (segment (start 53.7188 69.6368) (end 57.4209 65.9347) (width 0.25) (layer B.Cu) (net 28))
 (segment (start 57.4209 65.9347) (end 75.4168 65.9347) (width 0.25) (layer B.Cu) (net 28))
 (segment (start 75.4168 65.9347) (end 76.2247 66.7426) (width 0.25) (layer B.Cu) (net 28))
 (segment (start 76.2247 66.7426) (end 76.2247 67.11) (width 0.25) (layer B.Cu) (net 28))
 (segment (start 77.4 67.11) (end 76.2247 67.11) (width 0.25) (layer B.Cu) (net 28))
 (segment (start 56.73 72.53) (end 55.5047 72.53) (width 0.25) (layer F.Cu) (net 28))
 (segment (start 52 67.11) (end 52 68.2853) (width 0.25) (layer B.Cu) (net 28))
 (segment (start 55.5047 72.53) (end 53.7188 70.7441) (width 0.25) (layer F.Cu) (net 28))
 (segment (start 53.7188 70.7441) (end 53.7188 70.2204) (width 0.25) (layer F.Cu) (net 28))
 (via (at 53.7188 70.2204) (size 0.8) (layers F.Cu B.Cu) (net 28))
 (segment (start 55.5047 71.53) (end 54.8616 70.8869) (width 0.25) (layer F.Cu) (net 20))
 (segment (start 54.8616 70.8869) (end 54.8616 70.3039) (width 0.25) (layer F.Cu) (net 20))
 (segment (start 54.8616 70.3039) (end 53.1753 68.6176) (width 0.25) (layer F.Cu) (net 20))
 (segment (start 53.1753 68.6176) (end 53.1753 66.6193) (width 0.25) (layer F.Cu) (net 20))
 (segment (start 53.1753 66.6193) (end 52.3013 65.7453) (width 0.25) (layer F.Cu) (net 20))
 (segment (start 52.3013 65.7453) (end 52 65.7453) (width 0.25) (layer F.Cu) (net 20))
 (segment (start 53.1753 64.57) (end 54.3506 63.3947) (width 0.25) (layer B.Cu) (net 20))
 (segment (start 54.3506 63.3947) (end 75.4168 63.3947) (width 0.25) (layer B.Cu) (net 20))
 (segment (start 75.4168 63.3947) (end 76.2247 64.2026) (width 0.25) (layer B.Cu) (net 20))
 (segment (start 76.2247 64.2026) (end 76.2247 64.57) (width 0.25) (layer B.Cu) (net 20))
 (segment (start 77.4 64.57) (end 76.2247 64.57) (width 0.25) (layer B.Cu) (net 20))
 (segment (start 52 64.57) (end 53.1753 64.57) (width 0.25) (layer B.Cu) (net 20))
 (segment (start 52 64.57) (end 52 65.7453) (width 0.25) (layer F.Cu) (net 20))
 (segment (start 56.73 71.53) (end 55.5047 71.53) (width 0.25) (layer F.Cu) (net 20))
 (segment (start 55.5047 70.53) (end 55.5047 70.3101) (width 0.25) (layer F.Cu) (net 19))
 (segment (start 55.5047 70.3101) (end 53.6256 68.431) (width 0.25) (layer F.Cu) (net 19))
 (segment (start 53.6256 68.431) (end 53.6256 64.4635) (width 0.25) (layer F.Cu) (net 19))
 (segment (start 53.6256 64.4635) (end 52.3674 63.2053) (width 0.25) (layer F.Cu) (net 19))
 (segment (start 52.3674 63.2053) (end 52 63.2053) (width 0.25) (layer F.Cu) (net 19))
 (segment (start 77.4 62.03) (end 76.2247 62.03) (width 0.25) (layer B.Cu) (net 19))
 (segment (start 52 62.03) (end 53.1753 62.03) (width 0.25) (layer B.Cu) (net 19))
 (segment (start 53.1753 62.03) (end 54.3506 60.8547) (width 0.25) (layer B.Cu) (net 19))
 (segment (start 54.3506 60.8547) (end 75.4168 60.8547) (width 0.25) (layer B.Cu) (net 19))
 (segment (start 75.4168 60.8547) (end 76.2247 61.6626) (width 0.25) (layer B.Cu) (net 19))
 (segment (start 76.2247 61.6626) (end 76.2247 62.03) (width 0.25) (layer B.Cu) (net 19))
 (segment (start 52 62.03) (end 52 63.2053) (width 0.25) (layer F.Cu) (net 19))
 (segment (start 56.73 70.53) (end 55.5047 70.53) (width 0.25) (layer F.Cu) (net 19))
 (segment (start 77.4 59.49) (end 76.2247 59.49) (width 0.25) (layer B.Cu) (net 18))
 (segment (start 52 59.49) (end 53.1753 59.49) (width 0.25) (layer B.Cu) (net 18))
 (segment (start 53.1753 59.49) (end 54.3506 58.3147) (width 0.25) (layer B.Cu) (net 18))
 (segment (start 54.3506 58.3147) (end 75.4168 58.3147) (width 0.25) (layer B.Cu) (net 18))
 (segment (start 75.4168 58.3147) (end 76.2247 59.1226) (width 0.25) (layer B.Cu) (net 18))
 (segment (start 76.2247 59.1226) (end 76.2247 59.49) (width 0.25) (layer B.Cu) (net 18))
 (segment (start 55.5047 69.53) (end 54.0759 68.1012) (width 0.25) (layer F.Cu) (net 18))
 (segment (start 54.0759 68.1012) (end 54.0759 62.3739) (width 0.25) (layer F.Cu) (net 18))
 (segment (start 54.0759 62.3739) (end 52.3673 60.6653) (width 0.25) (layer F.Cu) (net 18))
 (segment (start 52.3673 60.6653) (end 52 60.6653) (width 0.25) (layer F.Cu) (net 18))
 (segment (start 52 59.49) (end 52 60.6653) (width 0.25) (layer F.Cu) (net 18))
 (segment (start 56.73 69.53) (end 55.5047 69.53) (width 0.25) (layer F.Cu) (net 18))
 (segment (start 55.5047 68.53) (end 54.5262 67.5515) (width 0.25) (layer F.Cu) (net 17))
 (segment (start 54.5262 67.5515) (end 54.5262 60.2842) (width 0.25) (layer F.Cu) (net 17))
 (segment (start 54.5262 60.2842) (end 52.3673 58.1253) (width 0.25) (layer F.Cu) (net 17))
 (segment (start 52.3673 58.1253) (end 52 58.1253) (width 0.25) (layer F.Cu) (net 17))
 (segment (start 52 56.95) (end 52 58.1253) (width 0.25) (layer F.Cu) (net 17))
 (segment (start 56.73 68.53) (end 55.5047 68.53) (width 0.25) (layer F.Cu) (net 17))
 (segment (start 77.4 56.95) (end 76.2247 56.95) (width 0.25) (layer B.Cu) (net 17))
 (segment (start 52 56.95) (end 53.1753 56.95) (width 0.25) (layer B.Cu) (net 17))
 (segment (start 53.1753 56.95) (end 54.3506 55.7747) (width 0.25) (layer B.Cu) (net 17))
 (segment (start 54.3506 55.7747) (end 75.4168 55.7747) (width 0.25) (layer B.Cu) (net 17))
 (segment (start 75.4168 55.7747) (end 76.2247 56.5826) (width 0.25) (layer B.Cu) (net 17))
 (segment (start 76.2247 56.5826) (end 76.2247 56.95) (width 0.25) (layer B.Cu) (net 17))
 (segment (start 71.53 66.53) (end 72.7726 66.53) (width 0.25) (layer F.Cu) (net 9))
 (segment (start 72.7726 66.53) (end 73.0325 66.7899) (width 0.25) (layer F.Cu) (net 9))
 (segment (start 74.86 68.4747) (end 74.5614 68.4747) (width 0.25) (layer B.Cu) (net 9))
 (segment (start 74.5614 68.4747) (end 73.0325 66.9458) (width 0.25) (layer B.Cu) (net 9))
 (segment (start 73.0325 66.9458) (end 73.0325 66.7899) (width 0.25) (layer B.Cu) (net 9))
 (segment (start 74.86 69.65) (end 74.86 68.4747) (width 0.25) (layer B.Cu) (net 9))
 (via (at 73.0325 66.7899) (size 0.8) (layers F.Cu B.Cu) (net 9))
 (segment (start 67.63 64.63) (end 68.0717 64.1883) (width 0.25) (layer F.Cu) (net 1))
 (segment (start 68.0717 64.1883) (end 71.9383 64.1883) (width 0.25) (layer F.Cu) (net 1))
 (segment (start 71.9383 64.1883) (end 74.86 67.11) (width 0.25) (layer F.Cu) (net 1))
 (segment (start 66.63 63.4047) (end 72.5194 63.4047) (width 0.25) (layer F.Cu) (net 2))
 (segment (start 72.5194 63.4047) (end 73.6847 64.57) (width 0.25) (layer F.Cu) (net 2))
 (segment (start 74.86 64.57) (end 73.6847 64.57) (width 0.25) (layer F.Cu) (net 2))
 (segment (start 66.63 64.63) (end 66.63 63.4047) (width 0.25) (layer F.Cu) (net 2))
 (segment (start 65.63 63.4047) (end 67.0047 62.03) (width 0.25) (layer F.Cu) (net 3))
 (segment (start 67.0047 62.03) (end 73.6847 62.03) (width 0.25) (layer F.Cu) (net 3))
 (segment (start 74.86 62.03) (end 73.6847 62.03) (width 0.25) (layer F.Cu) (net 3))
 (segment (start 65.63 64.63) (end 65.63 63.4047) (width 0.25) (layer F.Cu) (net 3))
 (segment (start 73.6847 59.49) (end 67.5447 59.49) (width 0.25) (layer F.Cu) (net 5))
 (segment (start 67.5447 59.49) (end 63.63 63.4047) (width 0.25) (layer F.Cu) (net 5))
 (segment (start 74.86 59.49) (end 73.6847 59.49) (width 0.25) (layer F.Cu) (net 5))
 (segment (start 63.63 64.63) (end 63.63 63.4047) (width 0.25) (layer F.Cu) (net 5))
 (segment (start 73.6847 56.95) (end 69.0847 56.95) (width 0.25) (layer F.Cu) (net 6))
 (segment (start 69.0847 56.95) (end 62.63 63.4047) (width 0.25) (layer F.Cu) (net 6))
 (segment (start 74.86 56.95) (end 73.6847 56.95) (width 0.25) (layer F.Cu) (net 6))
 (segment (start 62.63 64.63) (end 62.63 63.4047) (width 0.25) (layer F.Cu) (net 6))
 (segment (start 73.6847 54.41) (end 70.6247 54.41) (width 0.25) (layer F.Cu) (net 7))
 (segment (start 70.6247 54.41) (end 61.63 63.4047) (width 0.25) (layer F.Cu) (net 7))
 (segment (start 74.86 54.41) (end 73.6847 54.41) (width 0.25) (layer F.Cu) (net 7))
 (segment (start 61.63 64.63) (end 61.63 63.4047) (width 0.25) (layer F.Cu) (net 7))
 (segment (start 60.63 63.4047) (end 72.1647 51.87) (width 0.25) (layer F.Cu) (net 8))
 (segment (start 72.1647 51.87) (end 73.6847 51.87) (width 0.25) (layer F.Cu) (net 8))
 (segment (start 74.86 51.87) (end 73.6847 51.87) (width 0.25) (layer F.Cu) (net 8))
 (segment (start 60.63 64.63) (end 60.63 63.4047) (width 0.25) (layer F.Cu) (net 8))
 (segment (start 52 84.89) (end 61.8953 84.89) (width 0.25) (layer F.Cu) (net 25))
 (segment (start 61.8953 84.89) (end 65.63 81.1553) (width 0.25) (layer F.Cu) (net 25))
 (segment (start 65.63 81.1553) (end 70.54 86.0653) (width 0.25) (layer F.Cu) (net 25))
 (segment (start 70.54 86.0653) (end 75.4168 86.0653) (width 0.25) (layer F.Cu) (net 25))
 (segment (start 75.4168 86.0653) (end 76.2247 85.2574) (width 0.25) (layer F.Cu) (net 25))
 (segment (start 76.2247 85.2574) (end 76.2247 84.89) (width 0.25) (layer F.Cu) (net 25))
 (segment (start 77.4 84.89) (end 76.2247 84.89) (width 0.25) (layer F.Cu) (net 25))
 (segment (start 65.63 79.93) (end 65.63 81.1553) (width 0.25) (layer F.Cu) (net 25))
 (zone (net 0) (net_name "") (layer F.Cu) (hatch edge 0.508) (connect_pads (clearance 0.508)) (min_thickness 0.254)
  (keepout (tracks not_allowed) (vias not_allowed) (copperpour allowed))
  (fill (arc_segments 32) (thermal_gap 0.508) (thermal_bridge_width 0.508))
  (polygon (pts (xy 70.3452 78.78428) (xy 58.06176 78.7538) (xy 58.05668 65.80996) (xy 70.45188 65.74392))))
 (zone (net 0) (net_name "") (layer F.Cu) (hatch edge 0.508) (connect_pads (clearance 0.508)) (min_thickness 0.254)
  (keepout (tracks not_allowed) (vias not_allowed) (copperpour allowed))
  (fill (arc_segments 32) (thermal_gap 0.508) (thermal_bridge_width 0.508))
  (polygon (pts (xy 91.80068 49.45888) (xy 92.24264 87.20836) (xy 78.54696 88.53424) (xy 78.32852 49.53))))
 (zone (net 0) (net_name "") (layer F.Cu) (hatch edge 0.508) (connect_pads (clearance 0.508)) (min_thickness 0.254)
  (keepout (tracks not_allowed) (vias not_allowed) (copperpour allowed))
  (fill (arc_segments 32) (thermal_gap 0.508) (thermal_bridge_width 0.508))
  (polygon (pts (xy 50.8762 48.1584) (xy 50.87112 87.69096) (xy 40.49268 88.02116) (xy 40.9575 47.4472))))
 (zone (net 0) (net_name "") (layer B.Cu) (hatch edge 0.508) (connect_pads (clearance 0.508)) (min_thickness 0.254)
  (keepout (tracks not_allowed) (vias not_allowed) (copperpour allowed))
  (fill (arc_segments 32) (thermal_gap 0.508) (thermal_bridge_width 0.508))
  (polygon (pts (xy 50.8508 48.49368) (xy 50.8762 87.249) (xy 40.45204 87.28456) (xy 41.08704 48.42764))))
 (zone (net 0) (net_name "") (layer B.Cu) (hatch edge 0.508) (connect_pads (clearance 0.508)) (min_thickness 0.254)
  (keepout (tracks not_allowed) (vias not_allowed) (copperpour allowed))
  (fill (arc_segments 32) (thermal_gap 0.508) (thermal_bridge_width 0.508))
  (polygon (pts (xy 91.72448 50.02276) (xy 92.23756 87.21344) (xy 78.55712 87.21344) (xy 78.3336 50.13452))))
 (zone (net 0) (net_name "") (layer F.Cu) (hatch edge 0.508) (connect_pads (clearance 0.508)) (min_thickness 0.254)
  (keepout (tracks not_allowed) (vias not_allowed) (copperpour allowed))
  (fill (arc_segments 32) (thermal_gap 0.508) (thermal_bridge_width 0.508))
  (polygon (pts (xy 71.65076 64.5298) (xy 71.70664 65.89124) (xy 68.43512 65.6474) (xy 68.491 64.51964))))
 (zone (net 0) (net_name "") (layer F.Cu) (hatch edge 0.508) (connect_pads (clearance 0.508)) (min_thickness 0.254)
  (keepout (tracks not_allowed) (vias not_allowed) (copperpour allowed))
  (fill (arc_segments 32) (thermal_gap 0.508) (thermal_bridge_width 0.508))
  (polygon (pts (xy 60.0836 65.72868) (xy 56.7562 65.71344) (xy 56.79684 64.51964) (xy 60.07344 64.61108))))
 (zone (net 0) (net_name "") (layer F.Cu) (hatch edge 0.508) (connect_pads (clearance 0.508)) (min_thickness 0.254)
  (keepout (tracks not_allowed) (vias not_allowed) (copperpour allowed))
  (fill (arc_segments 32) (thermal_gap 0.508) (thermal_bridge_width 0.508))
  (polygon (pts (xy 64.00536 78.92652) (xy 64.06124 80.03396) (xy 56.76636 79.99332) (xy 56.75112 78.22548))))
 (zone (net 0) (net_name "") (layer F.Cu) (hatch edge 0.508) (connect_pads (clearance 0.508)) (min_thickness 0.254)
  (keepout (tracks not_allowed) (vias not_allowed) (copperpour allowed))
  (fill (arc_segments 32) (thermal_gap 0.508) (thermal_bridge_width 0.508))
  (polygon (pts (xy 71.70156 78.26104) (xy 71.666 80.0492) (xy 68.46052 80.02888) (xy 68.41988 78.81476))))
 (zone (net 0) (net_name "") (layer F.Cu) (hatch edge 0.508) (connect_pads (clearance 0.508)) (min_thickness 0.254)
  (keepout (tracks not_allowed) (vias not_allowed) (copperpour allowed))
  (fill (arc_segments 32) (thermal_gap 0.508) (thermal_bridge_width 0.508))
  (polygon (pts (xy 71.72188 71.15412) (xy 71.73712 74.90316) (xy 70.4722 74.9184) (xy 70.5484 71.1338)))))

